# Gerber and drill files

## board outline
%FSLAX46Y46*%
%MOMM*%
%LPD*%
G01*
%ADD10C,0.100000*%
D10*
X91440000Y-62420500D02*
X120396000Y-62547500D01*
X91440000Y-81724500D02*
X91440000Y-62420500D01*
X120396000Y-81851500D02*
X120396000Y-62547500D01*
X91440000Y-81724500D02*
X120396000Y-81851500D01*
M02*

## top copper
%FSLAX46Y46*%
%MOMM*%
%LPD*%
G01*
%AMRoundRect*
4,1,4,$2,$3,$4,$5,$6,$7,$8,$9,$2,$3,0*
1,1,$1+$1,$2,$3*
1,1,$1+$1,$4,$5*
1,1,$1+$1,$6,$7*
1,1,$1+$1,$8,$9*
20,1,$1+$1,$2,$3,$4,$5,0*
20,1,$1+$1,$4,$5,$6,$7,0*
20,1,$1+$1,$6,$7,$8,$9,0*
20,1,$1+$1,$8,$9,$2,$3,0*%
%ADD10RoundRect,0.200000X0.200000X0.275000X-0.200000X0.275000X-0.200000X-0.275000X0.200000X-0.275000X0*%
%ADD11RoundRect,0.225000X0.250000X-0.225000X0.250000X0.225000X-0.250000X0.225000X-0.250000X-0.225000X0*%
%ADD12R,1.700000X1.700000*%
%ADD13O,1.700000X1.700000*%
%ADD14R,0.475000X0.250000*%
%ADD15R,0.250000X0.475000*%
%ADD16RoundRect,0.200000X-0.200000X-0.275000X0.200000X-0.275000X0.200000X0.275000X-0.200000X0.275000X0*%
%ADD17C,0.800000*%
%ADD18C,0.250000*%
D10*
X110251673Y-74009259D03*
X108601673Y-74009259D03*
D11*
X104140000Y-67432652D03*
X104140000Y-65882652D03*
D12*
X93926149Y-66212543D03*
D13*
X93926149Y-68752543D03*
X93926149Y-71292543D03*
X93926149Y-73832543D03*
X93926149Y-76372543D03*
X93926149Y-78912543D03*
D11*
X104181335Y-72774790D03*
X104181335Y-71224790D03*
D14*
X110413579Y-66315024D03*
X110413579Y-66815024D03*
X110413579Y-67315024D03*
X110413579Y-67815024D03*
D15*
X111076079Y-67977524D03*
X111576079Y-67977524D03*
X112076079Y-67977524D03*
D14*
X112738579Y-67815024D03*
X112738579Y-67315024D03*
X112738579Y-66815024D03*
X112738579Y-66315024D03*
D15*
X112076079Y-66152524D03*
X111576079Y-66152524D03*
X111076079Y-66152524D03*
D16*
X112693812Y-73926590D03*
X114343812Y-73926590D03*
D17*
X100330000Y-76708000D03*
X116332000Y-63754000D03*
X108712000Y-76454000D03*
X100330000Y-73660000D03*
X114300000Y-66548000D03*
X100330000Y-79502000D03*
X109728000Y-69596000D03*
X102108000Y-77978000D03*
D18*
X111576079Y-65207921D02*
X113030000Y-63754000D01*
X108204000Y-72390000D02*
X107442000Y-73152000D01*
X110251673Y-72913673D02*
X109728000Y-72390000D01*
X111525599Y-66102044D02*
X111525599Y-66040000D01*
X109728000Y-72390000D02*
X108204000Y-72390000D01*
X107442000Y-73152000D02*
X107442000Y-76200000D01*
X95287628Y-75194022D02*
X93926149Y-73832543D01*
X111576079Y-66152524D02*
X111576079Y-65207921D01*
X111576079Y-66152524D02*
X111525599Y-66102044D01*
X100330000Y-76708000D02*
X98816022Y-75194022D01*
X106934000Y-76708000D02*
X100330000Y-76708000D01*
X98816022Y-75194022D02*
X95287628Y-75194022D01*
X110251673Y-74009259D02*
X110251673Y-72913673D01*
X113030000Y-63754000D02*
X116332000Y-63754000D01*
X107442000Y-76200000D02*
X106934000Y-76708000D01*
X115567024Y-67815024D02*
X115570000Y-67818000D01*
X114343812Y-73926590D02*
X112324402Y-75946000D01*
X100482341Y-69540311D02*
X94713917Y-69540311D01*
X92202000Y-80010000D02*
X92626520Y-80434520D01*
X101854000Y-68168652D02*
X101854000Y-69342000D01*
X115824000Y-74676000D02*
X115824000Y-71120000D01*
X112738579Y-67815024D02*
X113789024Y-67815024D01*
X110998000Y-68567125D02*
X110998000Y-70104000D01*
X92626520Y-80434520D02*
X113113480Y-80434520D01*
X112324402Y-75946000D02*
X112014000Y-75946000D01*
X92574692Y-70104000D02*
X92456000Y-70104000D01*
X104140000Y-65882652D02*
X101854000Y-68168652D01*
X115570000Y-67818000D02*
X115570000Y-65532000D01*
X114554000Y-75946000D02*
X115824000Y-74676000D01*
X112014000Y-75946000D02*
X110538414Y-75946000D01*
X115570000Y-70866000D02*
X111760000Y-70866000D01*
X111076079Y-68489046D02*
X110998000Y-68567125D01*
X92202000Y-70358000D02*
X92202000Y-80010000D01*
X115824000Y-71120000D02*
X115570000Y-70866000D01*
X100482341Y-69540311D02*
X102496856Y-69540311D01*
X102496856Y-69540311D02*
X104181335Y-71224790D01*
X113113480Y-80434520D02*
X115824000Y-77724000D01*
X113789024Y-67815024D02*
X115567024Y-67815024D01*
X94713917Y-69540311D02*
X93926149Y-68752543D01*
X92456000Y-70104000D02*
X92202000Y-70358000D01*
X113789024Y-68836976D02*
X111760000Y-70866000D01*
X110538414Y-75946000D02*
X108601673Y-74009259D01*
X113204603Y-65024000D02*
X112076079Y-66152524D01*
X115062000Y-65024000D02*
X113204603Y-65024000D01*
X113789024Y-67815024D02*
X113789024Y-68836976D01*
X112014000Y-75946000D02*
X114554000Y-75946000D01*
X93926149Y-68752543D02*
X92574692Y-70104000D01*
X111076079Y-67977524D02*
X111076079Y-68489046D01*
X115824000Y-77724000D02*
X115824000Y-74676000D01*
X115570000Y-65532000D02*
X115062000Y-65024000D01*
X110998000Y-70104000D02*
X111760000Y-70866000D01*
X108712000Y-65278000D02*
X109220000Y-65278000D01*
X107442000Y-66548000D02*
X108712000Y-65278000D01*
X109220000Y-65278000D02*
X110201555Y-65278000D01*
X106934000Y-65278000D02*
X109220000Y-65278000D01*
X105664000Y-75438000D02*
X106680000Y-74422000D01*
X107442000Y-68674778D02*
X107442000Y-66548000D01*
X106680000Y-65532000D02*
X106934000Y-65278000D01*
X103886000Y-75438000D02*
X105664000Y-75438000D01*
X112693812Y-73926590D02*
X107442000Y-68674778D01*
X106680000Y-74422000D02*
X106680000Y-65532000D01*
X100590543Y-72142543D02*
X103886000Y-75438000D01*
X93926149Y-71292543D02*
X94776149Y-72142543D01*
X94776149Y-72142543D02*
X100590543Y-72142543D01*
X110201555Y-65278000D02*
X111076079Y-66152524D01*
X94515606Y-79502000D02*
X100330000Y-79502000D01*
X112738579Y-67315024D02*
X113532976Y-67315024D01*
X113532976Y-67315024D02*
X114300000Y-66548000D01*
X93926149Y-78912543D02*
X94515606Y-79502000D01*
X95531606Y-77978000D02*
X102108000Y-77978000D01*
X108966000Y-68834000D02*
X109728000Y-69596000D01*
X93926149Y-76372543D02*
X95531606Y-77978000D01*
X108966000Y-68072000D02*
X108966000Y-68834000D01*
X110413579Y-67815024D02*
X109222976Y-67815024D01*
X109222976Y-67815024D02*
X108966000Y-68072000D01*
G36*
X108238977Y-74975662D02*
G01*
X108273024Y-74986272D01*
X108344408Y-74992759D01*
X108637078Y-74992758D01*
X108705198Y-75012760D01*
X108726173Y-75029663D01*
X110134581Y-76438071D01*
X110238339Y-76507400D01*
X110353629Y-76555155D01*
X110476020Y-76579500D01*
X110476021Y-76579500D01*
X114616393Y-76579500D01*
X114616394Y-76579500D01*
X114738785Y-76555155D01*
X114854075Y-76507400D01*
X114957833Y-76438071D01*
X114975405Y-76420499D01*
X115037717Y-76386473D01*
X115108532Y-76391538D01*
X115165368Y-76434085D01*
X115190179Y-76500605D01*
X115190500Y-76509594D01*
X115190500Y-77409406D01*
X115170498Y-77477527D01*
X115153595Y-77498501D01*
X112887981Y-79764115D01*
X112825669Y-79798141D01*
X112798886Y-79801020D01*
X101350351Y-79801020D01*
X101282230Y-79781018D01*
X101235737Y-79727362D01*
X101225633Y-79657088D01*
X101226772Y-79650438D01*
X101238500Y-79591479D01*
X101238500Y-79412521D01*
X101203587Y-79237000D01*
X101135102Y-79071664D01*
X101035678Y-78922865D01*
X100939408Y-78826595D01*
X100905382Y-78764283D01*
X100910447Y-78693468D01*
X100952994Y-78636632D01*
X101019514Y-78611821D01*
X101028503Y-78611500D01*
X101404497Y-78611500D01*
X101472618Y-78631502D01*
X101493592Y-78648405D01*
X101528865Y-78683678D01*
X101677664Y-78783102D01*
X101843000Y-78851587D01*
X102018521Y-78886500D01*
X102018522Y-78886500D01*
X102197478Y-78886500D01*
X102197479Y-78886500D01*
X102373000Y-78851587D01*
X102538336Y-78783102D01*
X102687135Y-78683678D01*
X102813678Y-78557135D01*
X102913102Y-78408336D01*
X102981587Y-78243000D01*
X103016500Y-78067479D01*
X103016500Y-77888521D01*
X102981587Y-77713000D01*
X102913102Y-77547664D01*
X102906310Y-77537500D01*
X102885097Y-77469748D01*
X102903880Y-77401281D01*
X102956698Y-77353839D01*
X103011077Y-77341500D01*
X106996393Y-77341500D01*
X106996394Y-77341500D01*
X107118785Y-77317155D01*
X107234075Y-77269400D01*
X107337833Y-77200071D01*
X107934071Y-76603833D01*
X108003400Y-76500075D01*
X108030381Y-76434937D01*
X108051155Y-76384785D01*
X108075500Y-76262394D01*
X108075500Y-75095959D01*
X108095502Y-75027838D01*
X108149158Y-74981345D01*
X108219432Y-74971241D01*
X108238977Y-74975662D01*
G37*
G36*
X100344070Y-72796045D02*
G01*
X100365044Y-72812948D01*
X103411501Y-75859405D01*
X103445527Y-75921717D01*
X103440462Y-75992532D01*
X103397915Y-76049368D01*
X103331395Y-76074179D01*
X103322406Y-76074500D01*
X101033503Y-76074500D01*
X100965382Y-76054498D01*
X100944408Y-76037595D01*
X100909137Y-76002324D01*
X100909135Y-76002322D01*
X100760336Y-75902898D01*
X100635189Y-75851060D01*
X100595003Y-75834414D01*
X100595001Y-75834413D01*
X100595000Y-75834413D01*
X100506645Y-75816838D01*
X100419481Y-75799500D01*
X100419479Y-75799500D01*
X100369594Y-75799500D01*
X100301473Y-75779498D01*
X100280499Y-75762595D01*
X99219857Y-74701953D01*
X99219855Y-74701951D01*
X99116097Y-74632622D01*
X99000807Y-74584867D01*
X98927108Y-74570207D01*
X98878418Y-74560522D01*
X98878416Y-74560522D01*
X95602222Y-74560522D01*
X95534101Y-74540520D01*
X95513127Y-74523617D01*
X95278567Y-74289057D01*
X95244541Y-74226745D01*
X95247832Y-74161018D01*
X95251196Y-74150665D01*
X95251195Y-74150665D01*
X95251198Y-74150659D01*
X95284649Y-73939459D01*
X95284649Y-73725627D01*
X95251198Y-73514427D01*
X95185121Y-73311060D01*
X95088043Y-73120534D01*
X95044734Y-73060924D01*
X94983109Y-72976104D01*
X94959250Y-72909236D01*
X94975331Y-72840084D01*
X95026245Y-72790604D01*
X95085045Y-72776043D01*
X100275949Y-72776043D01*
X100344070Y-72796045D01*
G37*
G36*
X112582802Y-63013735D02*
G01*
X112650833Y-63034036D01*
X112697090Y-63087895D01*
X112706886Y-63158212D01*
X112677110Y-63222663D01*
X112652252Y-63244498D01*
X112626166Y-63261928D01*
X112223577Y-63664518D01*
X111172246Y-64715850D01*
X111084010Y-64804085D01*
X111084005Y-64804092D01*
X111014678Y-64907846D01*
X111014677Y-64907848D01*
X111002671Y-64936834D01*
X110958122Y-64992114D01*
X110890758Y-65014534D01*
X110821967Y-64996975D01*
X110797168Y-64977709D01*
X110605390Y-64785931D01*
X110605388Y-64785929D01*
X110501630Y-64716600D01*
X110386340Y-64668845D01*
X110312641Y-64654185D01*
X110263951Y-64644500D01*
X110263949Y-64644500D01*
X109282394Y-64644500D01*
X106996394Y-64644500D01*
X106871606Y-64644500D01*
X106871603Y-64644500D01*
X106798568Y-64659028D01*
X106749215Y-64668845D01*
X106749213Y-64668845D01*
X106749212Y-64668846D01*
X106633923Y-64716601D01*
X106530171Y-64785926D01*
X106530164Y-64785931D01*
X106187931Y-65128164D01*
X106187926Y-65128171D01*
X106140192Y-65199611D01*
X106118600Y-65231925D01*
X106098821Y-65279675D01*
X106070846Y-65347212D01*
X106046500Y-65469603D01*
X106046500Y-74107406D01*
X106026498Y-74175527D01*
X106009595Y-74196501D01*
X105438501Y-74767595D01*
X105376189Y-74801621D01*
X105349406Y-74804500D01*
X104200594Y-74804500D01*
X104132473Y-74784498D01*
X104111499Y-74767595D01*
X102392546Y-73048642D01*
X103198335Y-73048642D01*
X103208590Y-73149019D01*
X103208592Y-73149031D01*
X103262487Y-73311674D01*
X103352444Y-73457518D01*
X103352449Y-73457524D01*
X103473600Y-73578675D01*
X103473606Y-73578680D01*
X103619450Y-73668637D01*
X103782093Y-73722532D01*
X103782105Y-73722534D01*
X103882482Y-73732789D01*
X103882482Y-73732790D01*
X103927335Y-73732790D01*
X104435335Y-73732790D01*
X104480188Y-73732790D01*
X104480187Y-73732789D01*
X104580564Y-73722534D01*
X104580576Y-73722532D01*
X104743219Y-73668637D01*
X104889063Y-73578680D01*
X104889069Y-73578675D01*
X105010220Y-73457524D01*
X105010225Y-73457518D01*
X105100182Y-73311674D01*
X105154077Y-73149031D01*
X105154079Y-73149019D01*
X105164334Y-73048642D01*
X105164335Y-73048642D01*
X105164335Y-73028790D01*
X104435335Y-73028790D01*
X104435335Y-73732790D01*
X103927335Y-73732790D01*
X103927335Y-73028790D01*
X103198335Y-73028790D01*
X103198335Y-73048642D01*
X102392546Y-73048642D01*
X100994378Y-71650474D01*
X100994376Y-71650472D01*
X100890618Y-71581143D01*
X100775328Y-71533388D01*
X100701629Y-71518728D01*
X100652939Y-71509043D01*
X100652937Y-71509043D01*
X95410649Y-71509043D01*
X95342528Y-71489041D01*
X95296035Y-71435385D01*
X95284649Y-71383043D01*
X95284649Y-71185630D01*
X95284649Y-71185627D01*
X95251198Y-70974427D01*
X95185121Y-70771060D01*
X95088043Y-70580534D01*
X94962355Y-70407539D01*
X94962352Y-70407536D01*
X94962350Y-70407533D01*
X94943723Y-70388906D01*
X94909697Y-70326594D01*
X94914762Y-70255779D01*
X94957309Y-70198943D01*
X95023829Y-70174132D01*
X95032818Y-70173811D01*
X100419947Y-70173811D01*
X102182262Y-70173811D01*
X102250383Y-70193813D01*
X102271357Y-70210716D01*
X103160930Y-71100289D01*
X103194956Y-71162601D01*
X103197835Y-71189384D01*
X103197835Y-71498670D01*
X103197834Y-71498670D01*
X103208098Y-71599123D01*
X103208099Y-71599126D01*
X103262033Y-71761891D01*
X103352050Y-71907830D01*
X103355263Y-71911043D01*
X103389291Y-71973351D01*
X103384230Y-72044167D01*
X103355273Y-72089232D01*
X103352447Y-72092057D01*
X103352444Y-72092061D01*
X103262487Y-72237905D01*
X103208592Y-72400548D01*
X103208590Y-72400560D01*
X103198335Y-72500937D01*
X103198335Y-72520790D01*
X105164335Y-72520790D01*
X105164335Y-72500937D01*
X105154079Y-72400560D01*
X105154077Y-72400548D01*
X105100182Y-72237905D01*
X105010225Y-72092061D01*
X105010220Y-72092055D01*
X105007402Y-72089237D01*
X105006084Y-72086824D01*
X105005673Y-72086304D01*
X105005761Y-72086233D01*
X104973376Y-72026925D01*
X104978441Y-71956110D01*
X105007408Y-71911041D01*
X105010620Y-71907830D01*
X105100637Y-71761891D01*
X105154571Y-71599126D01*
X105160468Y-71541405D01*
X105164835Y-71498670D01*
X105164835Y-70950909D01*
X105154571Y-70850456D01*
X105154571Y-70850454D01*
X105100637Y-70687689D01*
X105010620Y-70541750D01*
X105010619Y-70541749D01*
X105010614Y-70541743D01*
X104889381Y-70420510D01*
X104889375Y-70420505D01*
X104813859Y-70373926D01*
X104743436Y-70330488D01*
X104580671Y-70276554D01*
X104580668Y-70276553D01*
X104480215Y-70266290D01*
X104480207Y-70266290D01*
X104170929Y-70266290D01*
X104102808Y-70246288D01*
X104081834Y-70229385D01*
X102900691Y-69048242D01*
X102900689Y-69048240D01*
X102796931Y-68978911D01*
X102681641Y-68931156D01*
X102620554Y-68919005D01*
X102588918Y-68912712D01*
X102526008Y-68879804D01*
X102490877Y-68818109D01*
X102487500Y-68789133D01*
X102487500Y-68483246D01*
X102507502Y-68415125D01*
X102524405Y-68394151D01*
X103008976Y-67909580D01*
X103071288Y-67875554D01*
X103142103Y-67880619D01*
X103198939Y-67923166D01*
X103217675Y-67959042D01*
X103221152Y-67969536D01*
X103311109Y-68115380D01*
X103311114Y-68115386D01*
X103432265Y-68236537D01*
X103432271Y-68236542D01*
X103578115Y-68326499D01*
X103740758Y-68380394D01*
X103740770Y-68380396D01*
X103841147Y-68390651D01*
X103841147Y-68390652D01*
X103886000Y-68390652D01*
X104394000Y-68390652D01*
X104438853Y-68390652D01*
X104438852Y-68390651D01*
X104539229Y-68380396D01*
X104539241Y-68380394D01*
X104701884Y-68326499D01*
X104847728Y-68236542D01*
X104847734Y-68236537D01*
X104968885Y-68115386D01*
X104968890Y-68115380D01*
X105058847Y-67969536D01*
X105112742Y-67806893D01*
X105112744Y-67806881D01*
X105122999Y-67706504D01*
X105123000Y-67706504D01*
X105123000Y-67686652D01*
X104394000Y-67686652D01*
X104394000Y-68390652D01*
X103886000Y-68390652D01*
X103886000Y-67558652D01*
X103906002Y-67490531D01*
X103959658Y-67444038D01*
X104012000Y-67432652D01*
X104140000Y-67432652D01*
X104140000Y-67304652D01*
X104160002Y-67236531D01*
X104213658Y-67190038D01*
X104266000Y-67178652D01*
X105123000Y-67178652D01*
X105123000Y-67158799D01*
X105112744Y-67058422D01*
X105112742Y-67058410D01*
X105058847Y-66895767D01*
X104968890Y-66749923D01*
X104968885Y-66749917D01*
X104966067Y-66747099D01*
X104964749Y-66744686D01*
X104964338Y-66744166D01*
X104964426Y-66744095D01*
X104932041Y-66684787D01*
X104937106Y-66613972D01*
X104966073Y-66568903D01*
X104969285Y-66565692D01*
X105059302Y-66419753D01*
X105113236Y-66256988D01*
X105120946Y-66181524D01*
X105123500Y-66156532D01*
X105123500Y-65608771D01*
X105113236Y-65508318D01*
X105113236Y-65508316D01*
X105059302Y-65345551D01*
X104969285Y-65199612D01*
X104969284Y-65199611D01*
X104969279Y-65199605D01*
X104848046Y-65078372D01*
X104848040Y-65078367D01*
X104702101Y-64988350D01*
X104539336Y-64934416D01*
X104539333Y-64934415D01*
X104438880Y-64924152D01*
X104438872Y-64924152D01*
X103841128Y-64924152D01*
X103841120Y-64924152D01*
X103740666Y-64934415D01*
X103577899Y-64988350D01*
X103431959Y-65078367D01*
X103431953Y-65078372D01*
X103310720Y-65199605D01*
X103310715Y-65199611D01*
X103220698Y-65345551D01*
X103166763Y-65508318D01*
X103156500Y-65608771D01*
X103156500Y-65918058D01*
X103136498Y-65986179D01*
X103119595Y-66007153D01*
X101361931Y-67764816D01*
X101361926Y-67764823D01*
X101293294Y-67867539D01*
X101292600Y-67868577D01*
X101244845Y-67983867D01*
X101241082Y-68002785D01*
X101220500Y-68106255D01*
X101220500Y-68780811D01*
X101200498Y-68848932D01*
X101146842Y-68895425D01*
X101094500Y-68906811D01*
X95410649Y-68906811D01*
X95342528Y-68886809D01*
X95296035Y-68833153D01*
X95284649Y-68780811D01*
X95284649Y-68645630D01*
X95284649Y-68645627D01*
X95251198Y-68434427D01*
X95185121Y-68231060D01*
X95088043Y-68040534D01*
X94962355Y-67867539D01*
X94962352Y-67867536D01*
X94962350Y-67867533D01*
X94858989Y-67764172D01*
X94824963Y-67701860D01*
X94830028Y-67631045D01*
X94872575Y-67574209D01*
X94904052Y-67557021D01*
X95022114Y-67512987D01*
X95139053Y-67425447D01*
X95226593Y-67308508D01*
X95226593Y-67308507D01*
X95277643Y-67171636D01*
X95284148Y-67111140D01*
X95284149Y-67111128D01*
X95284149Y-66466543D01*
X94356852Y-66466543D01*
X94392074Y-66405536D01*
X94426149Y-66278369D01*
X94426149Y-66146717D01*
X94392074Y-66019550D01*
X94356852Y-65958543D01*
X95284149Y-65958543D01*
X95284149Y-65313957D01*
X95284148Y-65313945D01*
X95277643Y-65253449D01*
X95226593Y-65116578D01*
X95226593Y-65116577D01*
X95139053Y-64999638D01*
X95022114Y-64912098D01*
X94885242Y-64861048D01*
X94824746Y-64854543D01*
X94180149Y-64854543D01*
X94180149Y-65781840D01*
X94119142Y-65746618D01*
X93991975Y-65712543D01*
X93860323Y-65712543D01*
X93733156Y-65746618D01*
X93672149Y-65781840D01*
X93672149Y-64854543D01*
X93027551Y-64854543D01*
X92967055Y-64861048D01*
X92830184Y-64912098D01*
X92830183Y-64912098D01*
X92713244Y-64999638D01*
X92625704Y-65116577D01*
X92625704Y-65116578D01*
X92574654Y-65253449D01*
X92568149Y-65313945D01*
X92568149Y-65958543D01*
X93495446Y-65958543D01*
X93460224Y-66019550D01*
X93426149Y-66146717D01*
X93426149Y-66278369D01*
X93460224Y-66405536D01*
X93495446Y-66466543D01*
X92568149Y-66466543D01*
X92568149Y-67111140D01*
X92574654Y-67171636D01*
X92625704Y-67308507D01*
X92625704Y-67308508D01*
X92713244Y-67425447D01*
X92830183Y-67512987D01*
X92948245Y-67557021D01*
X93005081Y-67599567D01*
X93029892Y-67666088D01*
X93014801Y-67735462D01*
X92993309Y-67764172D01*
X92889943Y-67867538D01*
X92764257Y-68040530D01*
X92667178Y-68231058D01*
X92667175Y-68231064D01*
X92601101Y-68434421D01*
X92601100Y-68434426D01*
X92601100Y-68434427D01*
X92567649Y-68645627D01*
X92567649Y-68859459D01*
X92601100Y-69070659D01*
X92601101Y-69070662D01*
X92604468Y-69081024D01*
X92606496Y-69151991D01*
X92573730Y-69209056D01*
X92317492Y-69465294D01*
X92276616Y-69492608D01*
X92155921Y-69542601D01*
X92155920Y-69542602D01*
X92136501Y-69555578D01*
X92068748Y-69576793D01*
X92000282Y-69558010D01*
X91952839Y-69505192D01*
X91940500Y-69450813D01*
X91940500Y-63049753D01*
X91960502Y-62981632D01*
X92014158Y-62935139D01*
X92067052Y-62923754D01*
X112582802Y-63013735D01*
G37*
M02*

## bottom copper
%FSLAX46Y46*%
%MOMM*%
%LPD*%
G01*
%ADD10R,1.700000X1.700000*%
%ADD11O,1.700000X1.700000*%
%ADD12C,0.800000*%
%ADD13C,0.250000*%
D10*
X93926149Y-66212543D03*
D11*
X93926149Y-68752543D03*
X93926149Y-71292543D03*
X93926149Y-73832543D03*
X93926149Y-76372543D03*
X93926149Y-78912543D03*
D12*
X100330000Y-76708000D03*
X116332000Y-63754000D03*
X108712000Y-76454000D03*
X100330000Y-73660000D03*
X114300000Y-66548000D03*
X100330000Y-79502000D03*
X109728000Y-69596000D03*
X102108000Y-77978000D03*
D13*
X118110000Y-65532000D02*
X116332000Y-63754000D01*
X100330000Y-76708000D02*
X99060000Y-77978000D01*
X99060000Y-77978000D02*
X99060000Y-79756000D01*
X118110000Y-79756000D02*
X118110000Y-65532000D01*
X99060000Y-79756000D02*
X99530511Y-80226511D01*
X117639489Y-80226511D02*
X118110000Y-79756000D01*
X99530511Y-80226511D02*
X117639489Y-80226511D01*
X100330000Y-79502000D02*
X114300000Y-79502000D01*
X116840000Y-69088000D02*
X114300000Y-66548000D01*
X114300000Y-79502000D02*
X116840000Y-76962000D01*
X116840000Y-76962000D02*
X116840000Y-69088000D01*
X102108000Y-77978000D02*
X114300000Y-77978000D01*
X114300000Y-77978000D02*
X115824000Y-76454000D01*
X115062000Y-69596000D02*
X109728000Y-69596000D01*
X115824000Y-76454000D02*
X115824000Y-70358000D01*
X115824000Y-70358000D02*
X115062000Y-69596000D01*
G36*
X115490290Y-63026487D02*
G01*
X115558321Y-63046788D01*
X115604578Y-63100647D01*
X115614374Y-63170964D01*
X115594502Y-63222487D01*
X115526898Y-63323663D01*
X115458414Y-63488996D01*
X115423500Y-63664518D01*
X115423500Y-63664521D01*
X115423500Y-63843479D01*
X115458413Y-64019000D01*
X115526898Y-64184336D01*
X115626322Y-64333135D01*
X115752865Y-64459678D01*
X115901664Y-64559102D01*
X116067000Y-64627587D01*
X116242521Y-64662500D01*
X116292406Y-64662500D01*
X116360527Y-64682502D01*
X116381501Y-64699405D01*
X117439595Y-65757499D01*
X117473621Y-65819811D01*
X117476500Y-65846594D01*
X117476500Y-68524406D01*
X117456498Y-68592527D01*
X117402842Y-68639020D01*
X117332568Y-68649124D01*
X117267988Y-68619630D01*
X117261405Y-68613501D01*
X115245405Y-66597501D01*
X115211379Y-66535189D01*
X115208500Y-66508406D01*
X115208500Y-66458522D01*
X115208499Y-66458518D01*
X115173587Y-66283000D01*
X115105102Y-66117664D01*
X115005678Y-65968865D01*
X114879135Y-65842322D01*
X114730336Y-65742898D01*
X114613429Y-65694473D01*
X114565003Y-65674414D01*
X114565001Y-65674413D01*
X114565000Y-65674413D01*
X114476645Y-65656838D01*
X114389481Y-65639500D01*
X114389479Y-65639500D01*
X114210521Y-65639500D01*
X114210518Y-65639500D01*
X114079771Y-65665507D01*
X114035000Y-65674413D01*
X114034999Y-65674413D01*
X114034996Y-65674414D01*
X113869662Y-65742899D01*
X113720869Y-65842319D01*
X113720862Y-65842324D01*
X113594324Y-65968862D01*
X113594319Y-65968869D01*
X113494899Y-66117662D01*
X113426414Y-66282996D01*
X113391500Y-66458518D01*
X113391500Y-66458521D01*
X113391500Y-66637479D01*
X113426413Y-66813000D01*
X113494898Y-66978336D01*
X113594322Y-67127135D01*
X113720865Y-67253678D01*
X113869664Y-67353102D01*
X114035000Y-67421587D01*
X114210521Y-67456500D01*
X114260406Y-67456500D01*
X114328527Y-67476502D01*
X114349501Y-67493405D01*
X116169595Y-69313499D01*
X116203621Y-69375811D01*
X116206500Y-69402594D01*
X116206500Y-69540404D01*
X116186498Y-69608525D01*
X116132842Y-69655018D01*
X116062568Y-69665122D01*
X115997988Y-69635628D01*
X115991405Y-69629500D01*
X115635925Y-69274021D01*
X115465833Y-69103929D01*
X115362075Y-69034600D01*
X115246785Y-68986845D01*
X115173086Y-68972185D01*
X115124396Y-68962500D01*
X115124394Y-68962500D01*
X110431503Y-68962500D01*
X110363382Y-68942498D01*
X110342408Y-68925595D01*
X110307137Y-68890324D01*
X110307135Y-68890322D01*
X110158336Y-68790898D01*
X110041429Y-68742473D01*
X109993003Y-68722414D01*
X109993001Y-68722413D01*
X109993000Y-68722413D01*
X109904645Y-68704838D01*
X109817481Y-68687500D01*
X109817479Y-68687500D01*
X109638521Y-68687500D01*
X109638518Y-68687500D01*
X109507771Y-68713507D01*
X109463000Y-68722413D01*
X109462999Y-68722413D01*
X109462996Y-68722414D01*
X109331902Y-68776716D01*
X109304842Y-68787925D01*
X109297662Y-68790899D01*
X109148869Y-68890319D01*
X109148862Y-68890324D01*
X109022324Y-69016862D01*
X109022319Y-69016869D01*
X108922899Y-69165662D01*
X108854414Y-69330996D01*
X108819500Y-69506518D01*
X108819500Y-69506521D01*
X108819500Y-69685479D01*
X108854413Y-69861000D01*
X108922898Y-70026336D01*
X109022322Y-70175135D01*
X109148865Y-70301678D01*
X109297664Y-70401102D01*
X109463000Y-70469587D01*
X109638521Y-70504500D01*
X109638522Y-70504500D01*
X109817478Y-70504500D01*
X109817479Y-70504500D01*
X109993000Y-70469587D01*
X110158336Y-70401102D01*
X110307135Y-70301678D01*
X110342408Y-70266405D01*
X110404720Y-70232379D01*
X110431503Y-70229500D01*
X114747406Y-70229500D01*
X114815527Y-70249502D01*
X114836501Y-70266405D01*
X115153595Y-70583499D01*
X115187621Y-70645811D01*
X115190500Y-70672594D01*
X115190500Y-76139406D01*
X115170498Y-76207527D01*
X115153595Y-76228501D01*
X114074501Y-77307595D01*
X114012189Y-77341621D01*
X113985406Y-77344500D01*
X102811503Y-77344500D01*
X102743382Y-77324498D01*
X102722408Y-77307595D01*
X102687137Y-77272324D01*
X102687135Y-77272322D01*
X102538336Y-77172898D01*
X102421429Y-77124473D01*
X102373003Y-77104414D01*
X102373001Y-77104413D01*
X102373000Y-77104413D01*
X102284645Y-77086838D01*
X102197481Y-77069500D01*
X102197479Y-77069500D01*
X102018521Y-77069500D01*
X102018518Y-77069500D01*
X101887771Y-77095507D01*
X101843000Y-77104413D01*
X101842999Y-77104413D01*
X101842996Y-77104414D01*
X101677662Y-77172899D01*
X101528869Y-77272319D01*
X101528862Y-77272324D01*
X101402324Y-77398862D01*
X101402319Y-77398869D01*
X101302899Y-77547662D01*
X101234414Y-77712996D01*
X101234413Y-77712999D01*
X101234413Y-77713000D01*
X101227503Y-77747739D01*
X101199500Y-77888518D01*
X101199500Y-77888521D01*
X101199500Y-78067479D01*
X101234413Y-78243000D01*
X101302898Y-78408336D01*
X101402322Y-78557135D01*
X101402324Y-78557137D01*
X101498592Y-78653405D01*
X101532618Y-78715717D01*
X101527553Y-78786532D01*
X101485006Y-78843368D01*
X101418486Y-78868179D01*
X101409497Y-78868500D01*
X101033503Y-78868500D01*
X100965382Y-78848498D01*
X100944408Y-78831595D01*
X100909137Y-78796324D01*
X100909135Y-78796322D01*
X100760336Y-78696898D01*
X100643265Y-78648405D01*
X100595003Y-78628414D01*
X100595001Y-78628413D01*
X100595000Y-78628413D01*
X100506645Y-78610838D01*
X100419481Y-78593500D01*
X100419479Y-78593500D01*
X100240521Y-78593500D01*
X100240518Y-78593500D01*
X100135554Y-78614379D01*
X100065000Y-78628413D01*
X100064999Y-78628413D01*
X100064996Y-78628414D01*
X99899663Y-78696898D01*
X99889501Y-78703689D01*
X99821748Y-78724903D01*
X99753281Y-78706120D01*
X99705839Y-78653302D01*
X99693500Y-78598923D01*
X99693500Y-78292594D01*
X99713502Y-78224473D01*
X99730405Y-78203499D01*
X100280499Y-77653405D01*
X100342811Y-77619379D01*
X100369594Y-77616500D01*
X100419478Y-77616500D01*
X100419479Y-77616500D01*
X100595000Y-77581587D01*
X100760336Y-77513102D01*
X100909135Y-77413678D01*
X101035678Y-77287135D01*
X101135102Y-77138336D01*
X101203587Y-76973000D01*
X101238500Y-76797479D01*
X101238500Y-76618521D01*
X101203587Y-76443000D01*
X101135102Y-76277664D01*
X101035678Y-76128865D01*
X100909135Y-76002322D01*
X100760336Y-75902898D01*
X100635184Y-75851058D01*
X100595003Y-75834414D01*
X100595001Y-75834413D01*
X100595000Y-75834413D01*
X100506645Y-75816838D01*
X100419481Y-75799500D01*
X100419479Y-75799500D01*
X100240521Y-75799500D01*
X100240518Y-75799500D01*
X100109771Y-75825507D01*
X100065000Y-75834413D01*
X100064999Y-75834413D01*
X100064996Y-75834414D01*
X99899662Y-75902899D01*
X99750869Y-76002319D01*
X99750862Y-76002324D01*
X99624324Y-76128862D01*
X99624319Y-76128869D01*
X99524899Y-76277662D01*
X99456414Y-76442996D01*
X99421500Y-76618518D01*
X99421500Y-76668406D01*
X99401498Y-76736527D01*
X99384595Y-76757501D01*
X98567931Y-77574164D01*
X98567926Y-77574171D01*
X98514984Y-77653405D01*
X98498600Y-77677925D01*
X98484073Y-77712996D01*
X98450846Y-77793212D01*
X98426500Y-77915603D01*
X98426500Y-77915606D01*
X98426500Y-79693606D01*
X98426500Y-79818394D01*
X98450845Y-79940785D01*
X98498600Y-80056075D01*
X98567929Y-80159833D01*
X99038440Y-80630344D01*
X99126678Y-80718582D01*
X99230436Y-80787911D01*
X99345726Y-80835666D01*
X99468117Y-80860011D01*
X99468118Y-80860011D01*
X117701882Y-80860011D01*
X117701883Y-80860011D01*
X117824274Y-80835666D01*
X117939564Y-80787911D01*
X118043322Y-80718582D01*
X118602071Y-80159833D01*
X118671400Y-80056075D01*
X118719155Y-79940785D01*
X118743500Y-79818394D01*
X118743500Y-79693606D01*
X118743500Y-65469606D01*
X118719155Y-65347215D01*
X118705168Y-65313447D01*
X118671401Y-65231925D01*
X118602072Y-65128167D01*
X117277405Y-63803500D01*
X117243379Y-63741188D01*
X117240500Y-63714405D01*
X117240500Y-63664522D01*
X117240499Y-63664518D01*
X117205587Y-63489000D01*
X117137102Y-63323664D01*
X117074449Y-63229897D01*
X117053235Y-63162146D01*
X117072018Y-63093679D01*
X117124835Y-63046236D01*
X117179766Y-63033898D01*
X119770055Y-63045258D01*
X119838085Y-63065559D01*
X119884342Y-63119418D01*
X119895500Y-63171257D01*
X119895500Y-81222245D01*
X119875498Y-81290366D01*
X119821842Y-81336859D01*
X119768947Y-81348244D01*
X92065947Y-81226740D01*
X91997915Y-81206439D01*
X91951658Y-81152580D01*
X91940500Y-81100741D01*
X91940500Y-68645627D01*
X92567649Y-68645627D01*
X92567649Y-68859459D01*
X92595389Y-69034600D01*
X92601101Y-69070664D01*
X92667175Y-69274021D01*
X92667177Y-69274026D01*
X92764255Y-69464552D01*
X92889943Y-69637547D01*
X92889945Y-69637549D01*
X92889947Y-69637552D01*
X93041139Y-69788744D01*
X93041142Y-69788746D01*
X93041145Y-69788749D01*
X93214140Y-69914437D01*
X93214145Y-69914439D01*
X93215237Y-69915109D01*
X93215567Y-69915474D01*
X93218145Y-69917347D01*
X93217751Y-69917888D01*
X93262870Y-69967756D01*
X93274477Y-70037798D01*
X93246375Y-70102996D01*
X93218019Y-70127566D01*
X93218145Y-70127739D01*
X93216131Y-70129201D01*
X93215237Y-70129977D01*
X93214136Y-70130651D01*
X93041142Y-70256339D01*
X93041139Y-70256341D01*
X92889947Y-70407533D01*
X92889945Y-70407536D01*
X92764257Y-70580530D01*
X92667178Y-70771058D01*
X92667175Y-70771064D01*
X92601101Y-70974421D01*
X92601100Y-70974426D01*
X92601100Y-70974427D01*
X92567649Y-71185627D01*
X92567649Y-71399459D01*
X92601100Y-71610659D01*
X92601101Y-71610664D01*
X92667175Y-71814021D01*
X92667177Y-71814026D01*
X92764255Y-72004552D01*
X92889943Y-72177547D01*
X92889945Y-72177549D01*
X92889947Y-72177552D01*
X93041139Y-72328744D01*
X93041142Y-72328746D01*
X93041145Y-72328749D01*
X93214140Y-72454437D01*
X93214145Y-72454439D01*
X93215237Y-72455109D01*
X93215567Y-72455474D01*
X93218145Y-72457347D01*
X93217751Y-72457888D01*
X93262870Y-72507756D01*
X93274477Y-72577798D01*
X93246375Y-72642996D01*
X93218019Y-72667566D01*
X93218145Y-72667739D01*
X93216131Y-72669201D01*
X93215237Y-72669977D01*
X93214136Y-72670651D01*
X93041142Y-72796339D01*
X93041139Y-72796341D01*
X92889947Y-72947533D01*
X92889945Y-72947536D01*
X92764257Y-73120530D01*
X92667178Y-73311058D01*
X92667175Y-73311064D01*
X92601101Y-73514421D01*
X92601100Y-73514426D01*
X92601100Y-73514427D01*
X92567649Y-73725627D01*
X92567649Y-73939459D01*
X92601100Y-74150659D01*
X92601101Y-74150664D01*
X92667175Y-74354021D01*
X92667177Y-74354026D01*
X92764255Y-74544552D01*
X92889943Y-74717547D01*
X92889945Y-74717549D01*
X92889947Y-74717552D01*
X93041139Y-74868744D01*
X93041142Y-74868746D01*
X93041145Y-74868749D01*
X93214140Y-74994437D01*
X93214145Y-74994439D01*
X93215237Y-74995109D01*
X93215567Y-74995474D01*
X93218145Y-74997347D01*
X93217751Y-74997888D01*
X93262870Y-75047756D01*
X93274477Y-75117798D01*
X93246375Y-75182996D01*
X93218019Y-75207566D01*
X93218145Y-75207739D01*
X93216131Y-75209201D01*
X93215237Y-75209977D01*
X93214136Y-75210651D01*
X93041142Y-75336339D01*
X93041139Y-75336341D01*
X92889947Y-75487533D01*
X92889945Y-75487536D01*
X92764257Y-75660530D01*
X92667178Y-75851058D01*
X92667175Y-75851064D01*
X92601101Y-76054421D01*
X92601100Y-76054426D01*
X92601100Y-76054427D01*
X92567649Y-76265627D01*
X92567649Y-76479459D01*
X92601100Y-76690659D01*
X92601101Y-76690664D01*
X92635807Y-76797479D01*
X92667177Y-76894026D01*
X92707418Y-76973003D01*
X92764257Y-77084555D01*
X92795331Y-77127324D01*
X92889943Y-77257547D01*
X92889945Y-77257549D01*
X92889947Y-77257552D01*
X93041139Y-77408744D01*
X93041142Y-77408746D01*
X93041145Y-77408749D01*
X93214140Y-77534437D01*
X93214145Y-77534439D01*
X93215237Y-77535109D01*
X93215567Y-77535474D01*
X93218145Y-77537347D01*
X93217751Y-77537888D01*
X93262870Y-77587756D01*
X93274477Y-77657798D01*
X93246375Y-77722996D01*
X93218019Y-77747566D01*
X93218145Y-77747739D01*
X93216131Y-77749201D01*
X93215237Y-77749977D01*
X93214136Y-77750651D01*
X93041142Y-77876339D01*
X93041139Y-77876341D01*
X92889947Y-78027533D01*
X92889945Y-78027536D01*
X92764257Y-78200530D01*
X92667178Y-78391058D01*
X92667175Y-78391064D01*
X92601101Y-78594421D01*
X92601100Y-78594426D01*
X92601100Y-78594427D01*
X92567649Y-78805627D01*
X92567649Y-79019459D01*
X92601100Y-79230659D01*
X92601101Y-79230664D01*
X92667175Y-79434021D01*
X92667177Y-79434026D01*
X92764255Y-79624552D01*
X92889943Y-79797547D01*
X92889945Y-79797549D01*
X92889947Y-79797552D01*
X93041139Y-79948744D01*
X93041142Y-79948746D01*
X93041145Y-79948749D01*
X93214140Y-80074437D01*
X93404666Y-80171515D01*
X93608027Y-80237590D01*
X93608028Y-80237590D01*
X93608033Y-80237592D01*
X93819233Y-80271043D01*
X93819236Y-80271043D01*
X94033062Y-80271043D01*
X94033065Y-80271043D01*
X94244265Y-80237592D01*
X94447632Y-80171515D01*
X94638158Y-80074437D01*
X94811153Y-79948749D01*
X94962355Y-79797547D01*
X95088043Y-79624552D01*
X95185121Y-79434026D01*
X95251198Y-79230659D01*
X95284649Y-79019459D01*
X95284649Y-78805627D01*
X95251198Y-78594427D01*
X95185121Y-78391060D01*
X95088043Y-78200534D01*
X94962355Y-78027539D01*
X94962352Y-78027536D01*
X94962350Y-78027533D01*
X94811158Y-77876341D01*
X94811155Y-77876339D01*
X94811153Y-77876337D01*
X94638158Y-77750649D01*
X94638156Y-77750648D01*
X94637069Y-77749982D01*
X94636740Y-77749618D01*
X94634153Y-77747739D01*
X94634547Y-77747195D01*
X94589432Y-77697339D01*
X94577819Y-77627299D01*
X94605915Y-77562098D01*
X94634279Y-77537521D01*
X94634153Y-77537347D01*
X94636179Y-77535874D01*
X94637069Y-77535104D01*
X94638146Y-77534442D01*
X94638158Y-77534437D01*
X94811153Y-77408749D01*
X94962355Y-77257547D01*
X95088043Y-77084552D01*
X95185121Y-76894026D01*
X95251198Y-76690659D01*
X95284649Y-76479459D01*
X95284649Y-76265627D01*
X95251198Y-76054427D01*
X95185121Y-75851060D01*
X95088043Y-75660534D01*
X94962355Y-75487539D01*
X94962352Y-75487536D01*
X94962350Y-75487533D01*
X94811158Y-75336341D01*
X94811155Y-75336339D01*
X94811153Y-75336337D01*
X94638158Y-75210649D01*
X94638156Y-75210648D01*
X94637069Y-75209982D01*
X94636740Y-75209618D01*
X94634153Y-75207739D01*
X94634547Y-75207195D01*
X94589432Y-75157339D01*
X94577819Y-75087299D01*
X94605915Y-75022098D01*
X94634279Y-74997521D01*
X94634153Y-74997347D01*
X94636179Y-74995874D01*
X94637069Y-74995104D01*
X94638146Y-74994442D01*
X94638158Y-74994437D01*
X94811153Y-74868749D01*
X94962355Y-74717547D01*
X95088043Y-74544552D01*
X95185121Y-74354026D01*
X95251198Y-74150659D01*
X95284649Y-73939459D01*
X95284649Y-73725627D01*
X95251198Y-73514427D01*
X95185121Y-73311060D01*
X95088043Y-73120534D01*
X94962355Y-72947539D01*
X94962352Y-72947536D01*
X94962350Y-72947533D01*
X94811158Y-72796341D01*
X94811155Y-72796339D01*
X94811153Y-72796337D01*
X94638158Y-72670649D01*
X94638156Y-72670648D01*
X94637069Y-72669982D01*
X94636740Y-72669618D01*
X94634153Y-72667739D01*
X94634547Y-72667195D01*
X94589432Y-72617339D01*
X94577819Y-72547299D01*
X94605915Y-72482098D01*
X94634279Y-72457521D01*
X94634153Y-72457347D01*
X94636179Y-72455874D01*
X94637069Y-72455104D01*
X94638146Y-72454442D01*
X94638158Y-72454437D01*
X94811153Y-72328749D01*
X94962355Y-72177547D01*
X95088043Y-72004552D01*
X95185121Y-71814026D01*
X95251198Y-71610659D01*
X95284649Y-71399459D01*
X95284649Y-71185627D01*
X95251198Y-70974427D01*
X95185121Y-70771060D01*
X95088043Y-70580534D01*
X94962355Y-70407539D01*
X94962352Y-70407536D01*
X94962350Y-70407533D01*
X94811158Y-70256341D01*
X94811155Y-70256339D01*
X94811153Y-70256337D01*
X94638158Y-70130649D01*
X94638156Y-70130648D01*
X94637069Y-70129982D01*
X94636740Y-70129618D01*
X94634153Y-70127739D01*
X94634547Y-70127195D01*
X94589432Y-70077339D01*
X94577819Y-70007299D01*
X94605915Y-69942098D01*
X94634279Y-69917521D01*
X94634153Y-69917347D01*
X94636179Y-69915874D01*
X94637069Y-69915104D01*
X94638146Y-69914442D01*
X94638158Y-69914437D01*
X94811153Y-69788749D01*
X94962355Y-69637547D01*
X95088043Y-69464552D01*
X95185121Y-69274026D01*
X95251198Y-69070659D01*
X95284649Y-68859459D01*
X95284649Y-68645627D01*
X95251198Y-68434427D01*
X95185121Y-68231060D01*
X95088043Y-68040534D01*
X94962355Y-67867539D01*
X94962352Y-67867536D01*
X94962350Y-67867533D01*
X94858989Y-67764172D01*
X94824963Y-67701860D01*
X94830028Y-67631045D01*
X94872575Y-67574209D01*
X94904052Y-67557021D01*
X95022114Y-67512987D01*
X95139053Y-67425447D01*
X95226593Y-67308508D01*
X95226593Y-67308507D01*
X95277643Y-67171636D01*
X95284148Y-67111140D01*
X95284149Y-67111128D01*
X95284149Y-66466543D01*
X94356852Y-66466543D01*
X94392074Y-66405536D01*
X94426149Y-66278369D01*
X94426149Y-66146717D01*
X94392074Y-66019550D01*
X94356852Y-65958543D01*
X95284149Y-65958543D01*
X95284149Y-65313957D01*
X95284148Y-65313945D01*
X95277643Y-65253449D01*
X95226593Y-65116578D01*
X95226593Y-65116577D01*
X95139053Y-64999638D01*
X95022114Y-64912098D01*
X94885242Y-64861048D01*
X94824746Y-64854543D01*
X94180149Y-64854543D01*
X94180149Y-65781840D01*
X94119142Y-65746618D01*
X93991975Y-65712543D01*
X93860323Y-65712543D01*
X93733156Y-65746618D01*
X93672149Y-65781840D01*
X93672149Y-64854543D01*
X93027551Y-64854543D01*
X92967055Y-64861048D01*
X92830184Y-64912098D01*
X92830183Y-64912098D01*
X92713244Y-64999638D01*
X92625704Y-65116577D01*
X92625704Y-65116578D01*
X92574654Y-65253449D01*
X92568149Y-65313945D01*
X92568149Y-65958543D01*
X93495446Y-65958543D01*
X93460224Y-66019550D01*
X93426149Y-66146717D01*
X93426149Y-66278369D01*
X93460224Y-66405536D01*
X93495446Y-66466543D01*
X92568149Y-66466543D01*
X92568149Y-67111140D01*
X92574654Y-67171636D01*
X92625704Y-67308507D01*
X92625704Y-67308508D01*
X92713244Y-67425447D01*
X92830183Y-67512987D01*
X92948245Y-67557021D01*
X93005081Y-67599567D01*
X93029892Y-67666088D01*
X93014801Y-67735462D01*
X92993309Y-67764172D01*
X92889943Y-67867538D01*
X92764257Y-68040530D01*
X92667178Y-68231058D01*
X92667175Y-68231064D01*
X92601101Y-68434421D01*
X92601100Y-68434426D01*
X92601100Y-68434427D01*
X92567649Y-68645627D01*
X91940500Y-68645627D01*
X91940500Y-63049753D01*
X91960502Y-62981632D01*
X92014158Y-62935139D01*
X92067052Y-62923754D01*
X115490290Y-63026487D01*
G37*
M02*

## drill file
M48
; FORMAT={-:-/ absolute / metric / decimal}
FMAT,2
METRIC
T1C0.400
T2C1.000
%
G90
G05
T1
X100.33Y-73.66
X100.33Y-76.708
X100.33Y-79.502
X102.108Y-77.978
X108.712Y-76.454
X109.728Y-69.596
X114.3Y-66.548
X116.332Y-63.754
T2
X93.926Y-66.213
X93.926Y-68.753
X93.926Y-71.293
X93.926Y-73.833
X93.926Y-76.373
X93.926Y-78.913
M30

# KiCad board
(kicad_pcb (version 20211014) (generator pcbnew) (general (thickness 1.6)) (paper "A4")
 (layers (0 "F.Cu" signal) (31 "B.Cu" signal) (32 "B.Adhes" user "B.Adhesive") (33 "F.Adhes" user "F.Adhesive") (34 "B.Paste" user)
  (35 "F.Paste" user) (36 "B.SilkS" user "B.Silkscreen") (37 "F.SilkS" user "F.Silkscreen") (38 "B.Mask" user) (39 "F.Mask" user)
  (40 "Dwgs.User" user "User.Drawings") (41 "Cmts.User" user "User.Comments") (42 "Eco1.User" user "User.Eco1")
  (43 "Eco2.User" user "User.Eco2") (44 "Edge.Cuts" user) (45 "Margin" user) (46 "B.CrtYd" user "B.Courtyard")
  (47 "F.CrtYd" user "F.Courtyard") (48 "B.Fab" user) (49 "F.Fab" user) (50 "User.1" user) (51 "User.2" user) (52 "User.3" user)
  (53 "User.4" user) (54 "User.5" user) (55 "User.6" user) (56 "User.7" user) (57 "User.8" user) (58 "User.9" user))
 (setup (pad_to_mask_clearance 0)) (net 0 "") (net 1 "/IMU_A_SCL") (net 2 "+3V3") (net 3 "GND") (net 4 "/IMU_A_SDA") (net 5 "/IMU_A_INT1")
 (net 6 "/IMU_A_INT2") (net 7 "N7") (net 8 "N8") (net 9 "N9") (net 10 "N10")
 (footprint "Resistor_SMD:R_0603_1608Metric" (layer "F.Cu") (at 109.426673 74.009259 180)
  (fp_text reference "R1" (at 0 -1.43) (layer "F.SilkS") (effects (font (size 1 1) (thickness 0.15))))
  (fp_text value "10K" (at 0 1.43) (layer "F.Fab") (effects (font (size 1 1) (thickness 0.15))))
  (pad "1" smd roundrect (at -0.825 0 180) (size 0.8 0.95) (layers "F.Cu" "F.Paste" "F.Mask") (roundrect_rratio 0.25) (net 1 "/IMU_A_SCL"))
  (pad "2" smd roundrect (at 0.825 0 180) (size 0.8 0.95) (layers "F.Cu" "F.Paste" "F.Mask") (roundrect_rratio 0.25) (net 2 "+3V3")))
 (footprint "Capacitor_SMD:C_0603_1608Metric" (layer "F.Cu") (at 104.14 66.657652 90)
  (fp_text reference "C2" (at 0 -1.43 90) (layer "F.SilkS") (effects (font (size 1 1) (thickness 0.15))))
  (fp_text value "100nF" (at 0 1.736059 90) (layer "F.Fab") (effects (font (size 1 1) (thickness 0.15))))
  (pad "1" smd roundrect (at -0.775 0 90) (size 0.9 0.95) (layers "F.Cu" "F.Paste" "F.Mask") (roundrect_rratio 0.25) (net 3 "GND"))
  (pad "2" smd roundrect (at 0.775 0 90) (size 0.9 0.95) (layers "F.Cu" "F.Paste" "F.Mask") (roundrect_rratio 0.25) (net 2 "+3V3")))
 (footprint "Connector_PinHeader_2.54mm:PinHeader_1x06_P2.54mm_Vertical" (layer "F.Cu") (at 93.926149 66.212543)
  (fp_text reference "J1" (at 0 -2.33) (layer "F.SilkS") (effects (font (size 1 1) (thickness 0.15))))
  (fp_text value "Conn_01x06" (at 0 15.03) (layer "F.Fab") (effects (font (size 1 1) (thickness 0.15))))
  (pad "1" thru_hole rect (at 0 0) (size 1.7 1.7) (drill 1) (layers *.Cu *.Mask) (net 3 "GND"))
  (pad "2" thru_hole oval (at 0 2.54) (size 1.7 1.7) (drill 1) (layers *.Cu *.Mask) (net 2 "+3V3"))
  (pad "3" thru_hole oval (at 0 5.08) (size 1.7 1.7) (drill 1) (layers *.Cu *.Mask) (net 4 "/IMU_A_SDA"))
  (pad "4" thru_hole oval (at 0 7.62) (size 1.7 1.7) (drill 1) (layers *.Cu *.Mask) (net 1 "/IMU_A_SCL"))
  (pad "5" thru_hole oval (at 0 10.16) (size 1.7 1.7) (drill 1) (layers *.Cu *.Mask) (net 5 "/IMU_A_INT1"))
  (pad "6" thru_hole oval (at 0 12.7) (size 1.7 1.7) (drill 1) (layers *.Cu *.Mask) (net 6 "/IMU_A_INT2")))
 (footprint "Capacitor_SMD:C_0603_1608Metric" (layer "F.Cu") (at 104.181335 71.99979 90)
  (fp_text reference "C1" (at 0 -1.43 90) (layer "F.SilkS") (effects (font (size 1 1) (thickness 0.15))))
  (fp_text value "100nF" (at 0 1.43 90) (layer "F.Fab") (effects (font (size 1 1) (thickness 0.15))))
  (pad "1" smd roundrect (at -0.775 0 90) (size 0.9 0.95) (layers "F.Cu" "F.Paste" "F.Mask") (roundrect_rratio 0.25) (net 3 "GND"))
  (pad "2" smd roundrect (at 0.775 0 90) (size 0.9 0.95) (layers "F.Cu" "F.Paste" "F.Mask") (roundrect_rratio 0.25) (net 2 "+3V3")))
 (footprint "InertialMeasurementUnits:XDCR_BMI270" (layer "F.Cu") (at 111.576079 67.065024)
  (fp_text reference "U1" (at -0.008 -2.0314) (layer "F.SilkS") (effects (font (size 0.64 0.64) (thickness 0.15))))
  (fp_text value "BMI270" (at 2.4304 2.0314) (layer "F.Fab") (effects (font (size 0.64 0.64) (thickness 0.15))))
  (pad "1" smd rect locked (at -1.1625 -0.75) (size 0.475 0.25) (layers "F.Cu" "F.Paste" "F.Mask") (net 3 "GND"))
  (pad "2" smd rect locked (at -1.1625 -0.25) (size 0.475 0.25) (layers "F.Cu" "F.Paste" "F.Mask") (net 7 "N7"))
  (pad "3" smd rect locked (at -1.1625 0.25) (size 0.475 0.25) (layers "F.Cu" "F.Paste" "F.Mask") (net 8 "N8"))
  (pad "4" smd rect locked (at -1.1625 0.75) (size 0.475 0.25) (layers "F.Cu" "F.Paste" "F.Mask") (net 5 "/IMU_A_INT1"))
  (pad "5" smd rect locked (at -0.5 0.9125) (size 0.25 0.475) (layers "F.Cu" "F.Paste" "F.Mask") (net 2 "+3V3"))
  (pad "6" smd rect locked (at 0 0.9125) (size 0.25 0.475) (layers "F.Cu" "F.Paste" "F.Mask") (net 3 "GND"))
  (pad "7" smd rect locked (at 0.5 0.9125) (size 0.25 0.475) (layers "F.Cu" "F.Paste" "F.Mask") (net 3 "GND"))
  (pad "8" smd rect locked (at 1.1625 0.75) (size 0.475 0.25) (layers "F.Cu" "F.Paste" "F.Mask") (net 2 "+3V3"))
  (pad "9" smd rect locked (at 1.1625 0.25) (size 0.475 0.25) (layers "F.Cu" "F.Paste" "F.Mask") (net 6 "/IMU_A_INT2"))
  (pad "10" smd rect locked (at 1.1625 -0.25) (size 0.475 0.25) (layers "F.Cu" "F.Paste" "F.Mask") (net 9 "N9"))
  (pad "11" smd rect locked (at 1.1625 -0.75) (size 0.475 0.25) (layers "F.Cu" "F.Paste" "F.Mask") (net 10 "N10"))
  (pad "12" smd rect locked (at 0.5 -0.9125) (size 0.25 0.475) (layers "F.Cu" "F.Paste" "F.Mask") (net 2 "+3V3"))
  (pad "13" smd rect locked (at 0 -0.9125) (size 0.25 0.475) (layers "F.Cu" "F.Paste" "F.Mask") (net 1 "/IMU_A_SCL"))
  (pad "14" smd rect locked (at -0.5 -0.9125) (size 0.25 0.475) (layers "F.Cu" "F.Paste" "F.Mask") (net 4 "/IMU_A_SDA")))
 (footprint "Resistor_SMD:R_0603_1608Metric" (layer "F.Cu") (at 113.518812 73.92659)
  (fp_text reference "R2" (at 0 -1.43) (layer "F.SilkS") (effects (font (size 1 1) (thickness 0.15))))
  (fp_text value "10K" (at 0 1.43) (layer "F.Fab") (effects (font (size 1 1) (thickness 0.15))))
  (pad "1" smd roundrect (at -0.825 0) (size 0.8 0.95) (layers "F.Cu" "F.Paste" "F.Mask") (roundrect_rratio 0.25) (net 4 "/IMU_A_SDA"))
  (pad "2" smd roundrect (at 0.825 0) (size 0.8 0.95) (layers "F.Cu" "F.Paste" "F.Mask") (roundrect_rratio 0.25) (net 2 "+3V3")))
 (gr_line (start 91.44 62.4205) (end 120.396 62.5475) (layer "Edge.Cuts") (width 0.1))
 (gr_line (start 91.44 81.7245) (end 91.44 62.4205) (layer "Edge.Cuts") (width 0.1))
 (gr_line (start 120.396 81.8515) (end 120.396 62.5475) (layer "Edge.Cuts") (width 0.1))
 (gr_line (start 91.44 81.7245) (end 120.396 81.8515) (layer "Edge.Cuts") (width 0.1))
 (segment (start 111.576079 65.207921) (end 113.03 63.754) (width 0.25) (layer "F.Cu") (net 1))
 (segment (start 108.204 72.39) (end 107.442 73.152) (width 0.25) (layer "F.Cu") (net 1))
 (segment (start 110.251673 72.913673) (end 109.728 72.39) (width 0.25) (layer "F.Cu") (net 1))
 (segment (start 111.525599 66.102044) (end 111.525599 66.04) (width 0.25) (layer "F.Cu") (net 1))
 (segment (start 109.728 72.39) (end 108.204 72.39) (width 0.25) (layer "F.Cu") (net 1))
 (segment (start 107.442 73.152) (end 107.442 76.2) (width 0.25) (layer "F.Cu") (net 1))
 (segment (start 95.287628 75.194022) (end 93.926149 73.832543) (width 0.25) (layer "F.Cu") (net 1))
 (segment (start 111.576079 66.152524) (end 111.576079 65.207921) (width 0.25) (layer "F.Cu") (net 1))
 (segment (start 111.576079 66.152524) (end 111.525599 66.102044) (width 0.25) (layer "F.Cu") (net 1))
 (segment (start 100.33 76.708) (end 98.816022 75.194022) (width 0.25) (layer "F.Cu") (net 1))
 (segment (start 106.934 76.708) (end 100.33 76.708) (width 0.25) (layer "F.Cu") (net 1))
 (segment (start 98.816022 75.194022) (end 95.287628 75.194022) (width 0.25) (layer "F.Cu") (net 1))
 (segment (start 110.251673 74.009259) (end 110.251673 72.913673) (width 0.25) (layer "F.Cu") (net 1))
 (segment (start 113.03 63.754) (end 116.332 63.754) (width 0.25) (layer "F.Cu") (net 1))
 (segment (start 107.442 76.2) (end 106.934 76.708) (width 0.25) (layer "F.Cu") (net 1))
 (via (at 100.33 76.708) (size 0.8) (drill 0.4) (layers "F.Cu" "B.Cu") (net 1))
 (via (at 116.332 63.754) (size 0.8) (drill 0.4) (layers "F.Cu" "B.Cu") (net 1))
 (segment (start 118.11 65.532) (end 116.332 63.754) (width 0.25) (layer "B.Cu") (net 1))
 (segment (start 100.33 76.708) (end 99.06 77.978) (width 0.25) (layer "B.Cu") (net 1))
 (segment (start 99.06 77.978) (end 99.06 79.756) (width 0.25) (layer "B.Cu") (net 1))
 (segment (start 118.11 79.756) (end 118.11 65.532) (width 0.25) (layer "B.Cu") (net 1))
 (segment (start 99.06 79.756) (end 99.530511 80.226511) (width 0.25) (layer "B.Cu") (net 1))
 (segment (start 117.639489 80.226511) (end 118.11 79.756) (width 0.25) (layer "B.Cu") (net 1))
 (segment (start 99.530511 80.226511) (end 117.639489 80.226511) (width 0.25) (layer "B.Cu") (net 1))
 (segment (start 115.567024 67.815024) (end 115.57 67.818) (width 0.25) (layer "F.Cu") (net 2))
 (segment (start 114.343812 73.92659) (end 112.324402 75.946) (width 0.25) (layer "F.Cu") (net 2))
 (segment (start 100.482341 69.540311) (end 94.713917 69.540311) (width 0.25) (layer "F.Cu") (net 2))
 (segment (start 92.202 80.01) (end 92.62652 80.43452) (width 0.25) (layer "F.Cu") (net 2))
 (segment (start 101.854 68.168652) (end 101.854 69.342) (width 0.25) (layer "F.Cu") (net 2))
 (segment (start 115.824 74.676) (end 115.824 71.12) (width 0.25) (layer "F.Cu") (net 2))
 (segment (start 112.738579 67.815024) (end 113.789024 67.815024) (width 0.25) (layer "F.Cu") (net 2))
 (segment (start 110.998 68.567125) (end 110.998 70.104) (width 0.25) (layer "F.Cu") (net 2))
 (segment (start 92.62652 80.43452) (end 113.11348 80.43452) (width 0.25) (layer "F.Cu") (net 2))
 (segment (start 112.324402 75.946) (end 112.014 75.946) (width 0.25) (layer "F.Cu") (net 2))
 (segment (start 92.574692 70.104) (end 92.456 70.104) (width 0.25) (layer "F.Cu") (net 2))
 (segment (start 104.14 65.882652) (end 101.854 68.168652) (width 0.25) (layer "F.Cu") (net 2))
 (segment (start 115.57 67.818) (end 115.57 65.532) (width 0.25) (layer "F.Cu") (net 2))
 (segment (start 114.554 75.946) (end 115.824 74.676) (width 0.25) (layer "F.Cu") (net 2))
 (segment (start 112.014 75.946) (end 110.538414 75.946) (width 0.25) (layer "F.Cu") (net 2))
 (segment (start 115.57 70.866) (end 111.76 70.866) (width 0.25) (layer "F.Cu") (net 2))
 (segment (start 111.076079 68.489046) (end 110.998 68.567125) (width 0.25) (layer "F.Cu") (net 2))
 (segment (start 92.202 70.358) (end 92.202 80.01) (width 0.25) (layer "F.Cu") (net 2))
 (segment (start 115.824 71.12) (end 115.57 70.866) (width 0.25) (layer "F.Cu") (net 2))
 (segment (start 100.482341 69.540311) (end 102.496856 69.540311) (width 0.25) (layer "F.Cu") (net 2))
 (segment (start 102.496856 69.540311) (end 104.181335 71.22479) (width 0.25) (layer "F.Cu") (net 2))
 (segment (start 113.11348 80.43452) (end 115.824 77.724) (width 0.25) (layer "F.Cu") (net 2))
 (segment (start 113.789024 67.815024) (end 115.567024 67.815024) (width 0.25) (layer "F.Cu") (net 2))
 (segment (start 94.713917 69.540311) (end 93.926149 68.752543) (width 0.25) (layer "F.Cu") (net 2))
 (segment (start 92.456 70.104) (end 92.202 70.358) (width 0.25) (layer "F.Cu") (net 2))
 (segment (start 113.789024 68.836976) (end 111.76 70.866) (width 0.25) (layer "F.Cu") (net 2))
 (segment (start 110.538414 75.946) (end 108.601673 74.009259) (width 0.25) (layer "F.Cu") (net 2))
 (segment (start 113.204603 65.024) (end 112.076079 66.152524) (width 0.25) (layer "F.Cu") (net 2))
 (segment (start 115.062 65.024) (end 113.204603 65.024) (width 0.25) (layer "F.Cu") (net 2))
 (segment (start 113.789024 67.815024) (end 113.789024 68.836976) (width 0.25) (layer "F.Cu") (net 2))
 (segment (start 112.014 75.946) (end 114.554 75.946) (width 0.25) (layer "F.Cu") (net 2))
 (segment (start 93.926149 68.752543) (end 92.574692 70.104) (width 0.25) (layer "F.Cu") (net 2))
 (segment (start 111.076079 67.977524) (end 111.076079 68.489046) (width 0.25) (layer "F.Cu") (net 2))
 (segment (start 115.824 77.724) (end 115.824 74.676) (width 0.25) (layer "F.Cu") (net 2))
 (segment (start 115.57 65.532) (end 115.062 65.024) (width 0.25) (layer "F.Cu") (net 2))
 (segment (start 110.998 70.104) (end 111.76 70.866) (width 0.25) (layer "F.Cu") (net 2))
 (segment (start 108.712 65.278) (end 109.22 65.278) (width 0.25) (layer "F.Cu") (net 4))
 (segment (start 107.442 66.548) (end 108.712 65.278) (width 0.25) (layer "F.Cu") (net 4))
 (segment (start 109.22 65.278) (end 110.201555 65.278) (width 0.25) (layer "F.Cu") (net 4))
 (segment (start 106.934 65.278) (end 109.22 65.278) (width 0.25) (layer "F.Cu") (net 4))
 (segment (start 105.664 75.438) (end 106.68 74.422) (width 0.25) (layer "F.Cu") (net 4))
 (segment (start 107.442 68.674778) (end 107.442 66.548) (width 0.25) (layer "F.Cu") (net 4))
 (segment (start 106.68 65.532) (end 106.934 65.278) (width 0.25) (layer "F.Cu") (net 4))
 (segment (start 103.886 75.438) (end 105.664 75.438) (width 0.25) (layer "F.Cu") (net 4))
 (segment (start 112.693812 73.92659) (end 107.442 68.674778) (width 0.25) (layer "F.Cu") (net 4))
 (segment (start 106.68 74.422) (end 106.68 65.532) (width 0.25) (layer "F.Cu") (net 4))
 (segment (start 100.590543 72.142543) (end 103.886 75.438) (width 0.25) (layer "F.Cu") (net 4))
 (segment (start 93.926149 71.292543) (end 94.776149 72.142543) (width 0.25) (layer "F.Cu") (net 4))
 (segment (start 94.776149 72.142543) (end 100.590543 72.142543) (width 0.25) (layer "F.Cu") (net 4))
 (segment (start 110.201555 65.278) (end 111.076079 66.152524) (width 0.25) (layer "F.Cu") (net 4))
 (via (at 108.712 76.454) (size 0.8) (drill 0.4) (layers "F.Cu" "B.Cu") (free) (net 3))
 (via (at 100.33 73.66) (size 0.8) (drill 0.4) (layers "F.Cu" "B.Cu") (free) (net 3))
 (segment (start 94.515606 79.502) (end 100.33 79.502) (width 0.25) (layer "F.Cu") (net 6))
 (segment (start 112.738579 67.315024) (end 113.532976 67.315024) (width 0.25) (layer "F.Cu") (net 6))
 (segment (start 113.532976 67.315024) (end 114.3 66.548) (width 0.25) (layer "F.Cu") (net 6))
 (segment (start 93.926149 78.912543) (end 94.515606 79.502) (width 0.25) (layer "F.Cu") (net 6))
 (via (at 114.3 66.548) (size 0.8) (drill 0.4) (layers "F.Cu" "B.Cu") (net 6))
 (via (at 100.33 79.502) (size 0.8) (drill 0.4) (layers "F.Cu" "B.Cu") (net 6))
 (segment (start 100.33 79.502) (end 114.3 79.502) (width 0.25) (layer "B.Cu") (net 6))
 (segment (start 116.84 69.088) (end 114.3 66.548) (width 0.25) (layer "B.Cu") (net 6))
 (segment (start 114.3 79.502) (end 116.84 76.962) (width 0.25) (layer "B.Cu") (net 6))
 (segment (start 116.84 76.962) (end 116.84 69.088) (width 0.25) (layer "B.Cu") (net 6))
 (segment (start 95.531606 77.978) (end 102.108 77.978) (width 0.25) (layer "F.Cu") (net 5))
 (segment (start 108.966 68.834) (end 109.728 69.596) (width 0.25) (layer "F.Cu") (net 5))
 (segment (start 93.926149 76.372543) (end 95.531606 77.978) (width 0.25) (layer "F.Cu") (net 5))
 (segment (start 108.966 68.072) (end 108.966 68.834) (width 0.25) (layer "F.Cu") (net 5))
 (segment (start 110.413579 67.815024) (end 109.222976 67.815024) (width 0.25) (layer "F.Cu") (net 5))
 (segment (start 109.222976 67.815024) (end 108.966 68.072) (width 0.25) (layer "F.Cu") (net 5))
 (via (at 109.728 69.596) (size 0.8) (drill 0.4) (layers "F.Cu" "B.Cu") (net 5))
 (via (at 102.108 77.978) (size 0.8) (drill 0.4) (layers "F.Cu" "B.Cu") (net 5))
 (segment (start 102.108 77.978) (end 114.3 77.978) (width 0.25) (layer "B.Cu") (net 5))
 (segment (start 114.3 77.978) (end 115.824 76.454) (width 0.25) (layer "B.Cu") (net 5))
 (segment (start 115.062 69.596) (end 109.728 69.596) (width 0.25) (layer "B.Cu") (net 5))
 (segment (start 115.824 76.454) (end 115.824 70.358) (width 0.25) (layer "B.Cu") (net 5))
 (segment (start 115.824 70.358) (end 115.062 69.596) (width 0.25) (layer "B.Cu") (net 5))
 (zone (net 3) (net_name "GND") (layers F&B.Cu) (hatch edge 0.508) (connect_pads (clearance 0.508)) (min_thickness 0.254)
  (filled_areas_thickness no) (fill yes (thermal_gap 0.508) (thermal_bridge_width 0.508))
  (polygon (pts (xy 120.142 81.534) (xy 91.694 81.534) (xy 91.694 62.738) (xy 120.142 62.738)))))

